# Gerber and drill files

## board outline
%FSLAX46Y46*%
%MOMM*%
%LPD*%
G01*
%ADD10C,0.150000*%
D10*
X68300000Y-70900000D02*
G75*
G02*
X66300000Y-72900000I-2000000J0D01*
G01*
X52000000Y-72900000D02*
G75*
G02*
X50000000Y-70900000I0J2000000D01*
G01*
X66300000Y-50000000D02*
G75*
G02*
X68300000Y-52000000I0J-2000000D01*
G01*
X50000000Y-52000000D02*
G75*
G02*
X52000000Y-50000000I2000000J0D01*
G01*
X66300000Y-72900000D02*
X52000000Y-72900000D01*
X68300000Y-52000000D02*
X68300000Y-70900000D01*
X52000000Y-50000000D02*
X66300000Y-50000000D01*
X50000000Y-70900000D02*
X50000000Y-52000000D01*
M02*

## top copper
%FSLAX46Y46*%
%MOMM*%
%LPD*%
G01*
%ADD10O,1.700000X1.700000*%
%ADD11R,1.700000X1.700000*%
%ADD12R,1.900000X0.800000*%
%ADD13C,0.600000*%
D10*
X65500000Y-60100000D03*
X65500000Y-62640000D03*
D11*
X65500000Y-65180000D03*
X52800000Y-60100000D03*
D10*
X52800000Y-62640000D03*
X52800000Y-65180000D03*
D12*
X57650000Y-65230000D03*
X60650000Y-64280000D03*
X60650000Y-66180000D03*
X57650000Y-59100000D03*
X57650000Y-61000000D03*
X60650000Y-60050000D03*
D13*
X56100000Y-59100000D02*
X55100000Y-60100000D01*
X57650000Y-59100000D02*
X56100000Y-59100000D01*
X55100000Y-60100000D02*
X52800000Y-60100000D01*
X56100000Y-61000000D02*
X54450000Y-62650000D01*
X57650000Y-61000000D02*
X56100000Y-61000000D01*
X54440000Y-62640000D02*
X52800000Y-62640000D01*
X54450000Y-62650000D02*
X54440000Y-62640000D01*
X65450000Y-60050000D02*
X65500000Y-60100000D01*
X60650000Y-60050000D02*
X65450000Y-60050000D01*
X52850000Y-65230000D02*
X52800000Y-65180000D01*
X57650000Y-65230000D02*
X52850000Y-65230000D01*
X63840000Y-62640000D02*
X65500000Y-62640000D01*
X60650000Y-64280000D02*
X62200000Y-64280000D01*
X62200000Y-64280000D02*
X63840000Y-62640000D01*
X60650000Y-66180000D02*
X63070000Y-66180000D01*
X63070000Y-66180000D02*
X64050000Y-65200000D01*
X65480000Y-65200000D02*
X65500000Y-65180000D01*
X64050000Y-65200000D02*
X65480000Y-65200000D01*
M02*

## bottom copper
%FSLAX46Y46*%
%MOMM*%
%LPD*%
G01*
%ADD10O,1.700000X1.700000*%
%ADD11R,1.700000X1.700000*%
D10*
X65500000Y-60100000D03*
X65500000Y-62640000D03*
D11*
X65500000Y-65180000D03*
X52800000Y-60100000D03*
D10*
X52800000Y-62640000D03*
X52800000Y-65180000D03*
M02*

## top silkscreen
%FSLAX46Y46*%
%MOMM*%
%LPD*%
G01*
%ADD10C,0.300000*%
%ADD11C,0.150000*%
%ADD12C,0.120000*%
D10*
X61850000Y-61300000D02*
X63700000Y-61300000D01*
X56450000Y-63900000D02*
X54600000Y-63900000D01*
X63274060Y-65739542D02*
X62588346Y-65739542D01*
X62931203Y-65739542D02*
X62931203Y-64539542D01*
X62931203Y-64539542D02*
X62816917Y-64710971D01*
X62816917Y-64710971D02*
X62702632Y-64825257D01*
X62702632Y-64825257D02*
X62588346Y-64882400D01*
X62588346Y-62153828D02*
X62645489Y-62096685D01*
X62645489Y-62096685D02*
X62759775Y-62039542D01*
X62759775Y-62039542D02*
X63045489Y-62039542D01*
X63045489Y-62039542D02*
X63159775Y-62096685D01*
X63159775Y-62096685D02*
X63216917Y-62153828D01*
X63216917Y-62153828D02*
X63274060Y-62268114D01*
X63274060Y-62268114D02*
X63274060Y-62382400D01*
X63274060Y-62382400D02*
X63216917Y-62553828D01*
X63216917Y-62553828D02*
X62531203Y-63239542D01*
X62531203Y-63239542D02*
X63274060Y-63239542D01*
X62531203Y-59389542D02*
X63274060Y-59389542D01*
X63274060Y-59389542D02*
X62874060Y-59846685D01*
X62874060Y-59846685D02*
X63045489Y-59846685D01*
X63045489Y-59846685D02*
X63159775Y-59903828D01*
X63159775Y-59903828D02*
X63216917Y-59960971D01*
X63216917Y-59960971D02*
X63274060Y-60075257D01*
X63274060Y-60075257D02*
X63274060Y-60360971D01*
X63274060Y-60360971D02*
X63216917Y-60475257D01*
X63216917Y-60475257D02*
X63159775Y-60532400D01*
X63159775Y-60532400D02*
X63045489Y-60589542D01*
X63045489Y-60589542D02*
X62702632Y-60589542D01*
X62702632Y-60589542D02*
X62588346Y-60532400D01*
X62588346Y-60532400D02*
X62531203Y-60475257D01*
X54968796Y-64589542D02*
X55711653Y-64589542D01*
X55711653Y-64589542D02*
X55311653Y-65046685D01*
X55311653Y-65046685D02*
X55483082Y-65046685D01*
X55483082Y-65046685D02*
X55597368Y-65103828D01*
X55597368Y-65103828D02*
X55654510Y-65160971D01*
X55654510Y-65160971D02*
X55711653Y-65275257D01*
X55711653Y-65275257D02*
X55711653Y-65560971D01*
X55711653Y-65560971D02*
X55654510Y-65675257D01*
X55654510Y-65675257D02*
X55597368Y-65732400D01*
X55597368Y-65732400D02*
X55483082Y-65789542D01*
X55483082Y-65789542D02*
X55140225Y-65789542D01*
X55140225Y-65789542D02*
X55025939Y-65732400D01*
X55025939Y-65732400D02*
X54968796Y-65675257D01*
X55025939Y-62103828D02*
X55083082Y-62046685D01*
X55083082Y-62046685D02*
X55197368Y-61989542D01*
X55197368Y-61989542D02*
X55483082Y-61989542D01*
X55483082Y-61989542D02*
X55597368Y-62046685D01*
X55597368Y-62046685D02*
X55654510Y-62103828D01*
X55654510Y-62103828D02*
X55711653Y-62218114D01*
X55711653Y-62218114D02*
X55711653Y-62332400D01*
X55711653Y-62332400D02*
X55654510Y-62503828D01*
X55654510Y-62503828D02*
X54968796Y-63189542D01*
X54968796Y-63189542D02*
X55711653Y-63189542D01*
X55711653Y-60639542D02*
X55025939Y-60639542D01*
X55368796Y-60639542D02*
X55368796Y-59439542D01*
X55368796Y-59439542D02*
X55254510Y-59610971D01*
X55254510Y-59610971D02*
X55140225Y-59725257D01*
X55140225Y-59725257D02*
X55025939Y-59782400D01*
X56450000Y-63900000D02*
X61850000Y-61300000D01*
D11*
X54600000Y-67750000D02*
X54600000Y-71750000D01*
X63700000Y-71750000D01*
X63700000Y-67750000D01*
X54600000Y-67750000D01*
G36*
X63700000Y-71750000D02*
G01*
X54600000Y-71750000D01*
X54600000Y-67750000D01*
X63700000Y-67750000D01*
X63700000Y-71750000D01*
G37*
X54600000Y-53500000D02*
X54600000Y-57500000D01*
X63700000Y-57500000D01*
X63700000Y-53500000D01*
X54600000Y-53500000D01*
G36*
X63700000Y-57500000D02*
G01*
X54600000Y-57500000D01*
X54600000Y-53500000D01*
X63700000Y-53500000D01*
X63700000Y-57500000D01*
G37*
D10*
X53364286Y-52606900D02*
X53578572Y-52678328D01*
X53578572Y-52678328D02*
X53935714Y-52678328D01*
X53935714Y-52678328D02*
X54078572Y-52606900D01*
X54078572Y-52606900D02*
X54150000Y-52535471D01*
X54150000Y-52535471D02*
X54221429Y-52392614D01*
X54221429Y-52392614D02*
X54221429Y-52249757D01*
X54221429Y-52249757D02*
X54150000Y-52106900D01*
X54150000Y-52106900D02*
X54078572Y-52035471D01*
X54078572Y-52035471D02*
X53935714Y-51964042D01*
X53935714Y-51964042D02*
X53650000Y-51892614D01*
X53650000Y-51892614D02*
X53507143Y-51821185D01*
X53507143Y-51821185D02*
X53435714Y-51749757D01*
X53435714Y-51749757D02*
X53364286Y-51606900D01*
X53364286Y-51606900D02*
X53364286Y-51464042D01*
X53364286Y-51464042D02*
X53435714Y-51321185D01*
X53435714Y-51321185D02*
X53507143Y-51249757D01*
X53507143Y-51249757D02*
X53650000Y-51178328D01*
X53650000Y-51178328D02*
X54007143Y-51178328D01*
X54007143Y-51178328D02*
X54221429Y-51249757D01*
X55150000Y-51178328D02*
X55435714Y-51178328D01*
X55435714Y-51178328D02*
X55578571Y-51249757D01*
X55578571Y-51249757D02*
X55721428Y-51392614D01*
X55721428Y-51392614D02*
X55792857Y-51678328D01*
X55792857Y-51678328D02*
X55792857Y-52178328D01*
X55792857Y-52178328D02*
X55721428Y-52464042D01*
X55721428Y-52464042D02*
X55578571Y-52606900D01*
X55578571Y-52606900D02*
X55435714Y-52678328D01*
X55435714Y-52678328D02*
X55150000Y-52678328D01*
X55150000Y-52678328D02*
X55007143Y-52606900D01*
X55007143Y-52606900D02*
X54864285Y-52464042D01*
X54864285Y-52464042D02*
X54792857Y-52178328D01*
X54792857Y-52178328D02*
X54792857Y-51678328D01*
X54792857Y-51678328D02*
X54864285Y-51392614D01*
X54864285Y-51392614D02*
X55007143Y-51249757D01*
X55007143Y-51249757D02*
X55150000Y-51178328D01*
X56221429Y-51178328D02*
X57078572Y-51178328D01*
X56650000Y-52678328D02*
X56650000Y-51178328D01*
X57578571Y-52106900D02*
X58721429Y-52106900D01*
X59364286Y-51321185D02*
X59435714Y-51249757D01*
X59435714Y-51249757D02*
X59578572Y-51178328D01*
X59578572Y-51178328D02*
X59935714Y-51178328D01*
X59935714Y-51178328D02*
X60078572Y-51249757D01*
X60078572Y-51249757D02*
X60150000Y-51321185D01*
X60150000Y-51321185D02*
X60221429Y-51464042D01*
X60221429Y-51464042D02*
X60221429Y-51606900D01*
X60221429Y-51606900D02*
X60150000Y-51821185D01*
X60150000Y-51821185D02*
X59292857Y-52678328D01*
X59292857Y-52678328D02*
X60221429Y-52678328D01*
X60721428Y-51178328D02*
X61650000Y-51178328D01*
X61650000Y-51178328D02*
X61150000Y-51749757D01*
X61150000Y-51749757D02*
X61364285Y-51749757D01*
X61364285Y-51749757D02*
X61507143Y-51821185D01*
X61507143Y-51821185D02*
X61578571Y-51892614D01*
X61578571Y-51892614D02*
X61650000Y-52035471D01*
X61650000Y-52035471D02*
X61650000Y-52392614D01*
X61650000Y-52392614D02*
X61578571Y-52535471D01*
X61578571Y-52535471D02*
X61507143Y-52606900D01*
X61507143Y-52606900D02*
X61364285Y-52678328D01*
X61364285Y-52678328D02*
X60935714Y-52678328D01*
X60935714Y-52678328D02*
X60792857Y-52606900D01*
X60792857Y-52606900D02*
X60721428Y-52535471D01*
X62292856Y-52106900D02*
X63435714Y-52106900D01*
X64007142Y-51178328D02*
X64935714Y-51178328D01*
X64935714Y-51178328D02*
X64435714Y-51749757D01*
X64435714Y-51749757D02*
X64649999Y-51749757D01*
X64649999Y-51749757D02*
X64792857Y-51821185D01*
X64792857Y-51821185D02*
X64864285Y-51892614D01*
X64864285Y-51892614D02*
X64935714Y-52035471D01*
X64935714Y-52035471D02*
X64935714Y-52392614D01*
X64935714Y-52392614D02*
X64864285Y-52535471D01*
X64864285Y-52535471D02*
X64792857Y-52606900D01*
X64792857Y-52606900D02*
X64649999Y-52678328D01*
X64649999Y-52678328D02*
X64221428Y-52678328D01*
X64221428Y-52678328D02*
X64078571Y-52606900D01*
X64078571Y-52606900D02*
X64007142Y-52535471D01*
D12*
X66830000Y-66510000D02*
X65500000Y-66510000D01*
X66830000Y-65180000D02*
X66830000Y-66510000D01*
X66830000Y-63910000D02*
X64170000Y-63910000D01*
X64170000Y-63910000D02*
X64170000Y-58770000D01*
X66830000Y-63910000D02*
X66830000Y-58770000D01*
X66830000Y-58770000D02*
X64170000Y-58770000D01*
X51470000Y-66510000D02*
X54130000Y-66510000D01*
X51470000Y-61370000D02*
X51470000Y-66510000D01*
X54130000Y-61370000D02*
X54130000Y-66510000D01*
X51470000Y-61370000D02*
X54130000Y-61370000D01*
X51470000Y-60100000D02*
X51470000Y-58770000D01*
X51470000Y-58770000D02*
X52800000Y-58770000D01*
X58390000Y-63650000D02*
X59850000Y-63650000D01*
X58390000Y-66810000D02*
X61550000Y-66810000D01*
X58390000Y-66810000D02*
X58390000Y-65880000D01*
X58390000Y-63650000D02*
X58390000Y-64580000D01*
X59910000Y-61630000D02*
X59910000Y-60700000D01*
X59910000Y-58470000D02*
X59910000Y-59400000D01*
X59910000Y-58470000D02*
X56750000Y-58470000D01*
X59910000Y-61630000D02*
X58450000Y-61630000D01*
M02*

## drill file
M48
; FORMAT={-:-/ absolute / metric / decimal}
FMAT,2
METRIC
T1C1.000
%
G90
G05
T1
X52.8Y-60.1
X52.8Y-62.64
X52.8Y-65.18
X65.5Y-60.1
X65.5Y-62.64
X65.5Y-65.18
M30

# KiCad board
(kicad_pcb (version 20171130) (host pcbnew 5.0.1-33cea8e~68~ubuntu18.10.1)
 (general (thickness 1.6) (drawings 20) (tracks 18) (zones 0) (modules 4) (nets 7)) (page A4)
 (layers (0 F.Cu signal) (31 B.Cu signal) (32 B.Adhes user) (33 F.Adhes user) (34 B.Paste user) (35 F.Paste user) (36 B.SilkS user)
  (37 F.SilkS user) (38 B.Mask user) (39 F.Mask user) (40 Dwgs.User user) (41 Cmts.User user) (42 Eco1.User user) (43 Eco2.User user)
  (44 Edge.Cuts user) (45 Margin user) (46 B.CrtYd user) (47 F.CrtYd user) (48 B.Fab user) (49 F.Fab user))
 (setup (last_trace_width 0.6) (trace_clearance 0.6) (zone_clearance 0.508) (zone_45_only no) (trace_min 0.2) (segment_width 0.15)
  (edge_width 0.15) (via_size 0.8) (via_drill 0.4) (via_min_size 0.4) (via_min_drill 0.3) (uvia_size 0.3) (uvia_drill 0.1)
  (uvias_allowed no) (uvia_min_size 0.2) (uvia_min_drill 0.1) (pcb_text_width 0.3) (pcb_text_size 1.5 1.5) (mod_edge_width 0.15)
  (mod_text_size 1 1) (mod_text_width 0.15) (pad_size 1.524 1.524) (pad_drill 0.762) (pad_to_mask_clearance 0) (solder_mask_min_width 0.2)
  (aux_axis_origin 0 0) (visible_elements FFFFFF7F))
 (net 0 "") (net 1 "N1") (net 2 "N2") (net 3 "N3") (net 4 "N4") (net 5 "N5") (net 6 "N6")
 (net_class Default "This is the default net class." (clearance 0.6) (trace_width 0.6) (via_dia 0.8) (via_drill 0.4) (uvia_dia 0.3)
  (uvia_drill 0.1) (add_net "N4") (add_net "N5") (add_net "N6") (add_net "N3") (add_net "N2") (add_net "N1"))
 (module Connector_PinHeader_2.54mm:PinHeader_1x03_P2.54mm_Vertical (layer F.Cu) (at 65.5 65.18 180)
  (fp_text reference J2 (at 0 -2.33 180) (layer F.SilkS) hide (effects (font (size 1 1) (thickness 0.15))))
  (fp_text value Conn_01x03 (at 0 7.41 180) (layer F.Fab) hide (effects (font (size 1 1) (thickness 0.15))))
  (fp_line (start -1.33 -1.33) (end 0 -1.33) (layer F.SilkS) (width 0.12))
  (fp_line (start -1.33 0) (end -1.33 -1.33) (layer F.SilkS) (width 0.12))
  (fp_line (start -1.33 1.27) (end 1.33 1.27) (layer F.SilkS) (width 0.12))
  (fp_line (start 1.33 1.27) (end 1.33 6.41) (layer F.SilkS) (width 0.12))
  (fp_line (start -1.33 1.27) (end -1.33 6.41) (layer F.SilkS) (width 0.12))
  (fp_line (start -1.33 6.41) (end 1.33 6.41) (layer F.SilkS) (width 0.12))
  (pad 3 thru_hole oval (at 0 5.08 180) (size 1.7 1.7) (drill 1) (layers *.Cu *.Mask) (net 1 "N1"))
  (pad 2 thru_hole oval (at 0 2.54 180) (size 1.7 1.7) (drill 1) (layers *.Cu *.Mask) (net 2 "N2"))
  (pad 1 thru_hole rect (at 0 0 180) (size 1.7 1.7) (drill 1) (layers *.Cu *.Mask) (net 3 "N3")))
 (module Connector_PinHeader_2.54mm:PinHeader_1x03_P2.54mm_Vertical (layer F.Cu) (at 52.8 60.1)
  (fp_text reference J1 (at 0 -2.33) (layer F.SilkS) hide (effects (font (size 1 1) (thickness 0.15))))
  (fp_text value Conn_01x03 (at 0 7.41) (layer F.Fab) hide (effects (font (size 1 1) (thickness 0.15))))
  (fp_line (start -1.33 6.41) (end 1.33 6.41) (layer F.SilkS) (width 0.12))
  (fp_line (start -1.33 1.27) (end -1.33 6.41) (layer F.SilkS) (width 0.12))
  (fp_line (start 1.33 1.27) (end 1.33 6.41) (layer F.SilkS) (width 0.12))
  (fp_line (start -1.33 1.27) (end 1.33 1.27) (layer F.SilkS) (width 0.12))
  (fp_line (start -1.33 0) (end -1.33 -1.33) (layer F.SilkS) (width 0.12))
  (fp_line (start -1.33 -1.33) (end 0 -1.33) (layer F.SilkS) (width 0.12))
  (pad 1 thru_hole rect (at 0 0) (size 1.7 1.7) (drill 1) (layers *.Cu *.Mask) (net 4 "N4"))
  (pad 2 thru_hole oval (at 0 2.54) (size 1.7 1.7) (drill 1) (layers *.Cu *.Mask) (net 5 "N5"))
  (pad 3 thru_hole oval (at 0 5.08) (size 1.7 1.7) (drill 1) (layers *.Cu *.Mask) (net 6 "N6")))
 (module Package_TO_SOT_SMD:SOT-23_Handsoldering (layer F.Cu) (at 59.15 65.23 180)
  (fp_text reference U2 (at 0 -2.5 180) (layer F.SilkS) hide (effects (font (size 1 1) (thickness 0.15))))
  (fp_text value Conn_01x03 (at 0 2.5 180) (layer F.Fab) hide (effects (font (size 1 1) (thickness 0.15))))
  (fp_line (start 0.76 1.58) (end -0.7 1.58) (layer F.SilkS) (width 0.12))
  (fp_line (start 0.76 -1.58) (end -2.4 -1.58) (layer F.SilkS) (width 0.12))
  (fp_line (start 0.76 -1.58) (end 0.76 -0.65) (layer F.SilkS) (width 0.12))
  (fp_line (start 0.76 1.58) (end 0.76 0.65) (layer F.SilkS) (width 0.12))
  (pad 3 smd rect (at 1.5 0 180) (size 1.9 0.8) (layers F.Cu F.Paste F.Mask) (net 6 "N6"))
  (pad 2 smd rect (at -1.5 0.95 180) (size 1.9 0.8) (layers F.Cu F.Paste F.Mask) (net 2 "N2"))
  (pad 1 smd rect (at -1.5 -0.95 180) (size 1.9 0.8) (layers F.Cu F.Paste F.Mask) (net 3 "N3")))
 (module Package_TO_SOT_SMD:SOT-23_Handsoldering (layer F.Cu) (at 59.15 60.05)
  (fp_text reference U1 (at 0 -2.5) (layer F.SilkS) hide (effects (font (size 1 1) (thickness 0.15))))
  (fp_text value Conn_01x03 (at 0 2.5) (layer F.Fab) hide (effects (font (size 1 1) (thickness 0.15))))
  (fp_line (start 0.76 1.58) (end 0.76 0.65) (layer F.SilkS) (width 0.12))
  (fp_line (start 0.76 -1.58) (end 0.76 -0.65) (layer F.SilkS) (width 0.12))
  (fp_line (start 0.76 -1.58) (end -2.4 -1.58) (layer F.SilkS) (width 0.12))
  (fp_line (start 0.76 1.58) (end -0.7 1.58) (layer F.SilkS) (width 0.12))
  (pad 1 smd rect (at -1.5 -0.95) (size 1.9 0.8) (layers F.Cu F.Paste F.Mask) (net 4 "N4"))
  (pad 2 smd rect (at -1.5 0.95) (size 1.9 0.8) (layers F.Cu F.Paste F.Mask) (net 5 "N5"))
  (pad 3 smd rect (at 1.5 0) (size 1.9 0.8) (layers F.Cu F.Paste F.Mask) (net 1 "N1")))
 (gr_arc (start 66.3 70.9) (end 66.3 72.9) (angle -90) (layer Edge.Cuts) (width 0.15))
 (gr_arc (start 52 70.9) (end 50 70.9) (angle -90) (layer Edge.Cuts) (width 0.15))
 (gr_arc (start 66.3 52) (end 68.3 52) (angle -90) (layer Edge.Cuts) (width 0.15))
 (gr_arc (start 52 52) (end 52 50) (angle -90) (layer Edge.Cuts) (width 0.15))
 (gr_line (start 61.85 61.3) (end 63.7 61.3) (layer F.SilkS) (width 0.3))
 (gr_line (start 56.45 63.9) (end 54.6 63.9) (layer F.SilkS) (width 0.3))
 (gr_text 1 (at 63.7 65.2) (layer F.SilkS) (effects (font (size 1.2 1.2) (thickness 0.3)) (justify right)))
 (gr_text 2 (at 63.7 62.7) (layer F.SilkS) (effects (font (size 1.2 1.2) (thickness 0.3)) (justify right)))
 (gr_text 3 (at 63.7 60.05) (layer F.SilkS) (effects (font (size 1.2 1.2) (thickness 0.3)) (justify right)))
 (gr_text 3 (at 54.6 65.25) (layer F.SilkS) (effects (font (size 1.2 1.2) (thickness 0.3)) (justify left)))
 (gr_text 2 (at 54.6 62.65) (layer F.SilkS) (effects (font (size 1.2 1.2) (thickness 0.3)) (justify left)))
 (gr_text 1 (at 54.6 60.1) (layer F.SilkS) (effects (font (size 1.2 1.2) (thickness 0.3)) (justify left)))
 (gr_line (start 56.45 63.9) (end 61.85 61.3) (layer F.SilkS) (width 0.3))
 (gr_line (start 66.3 72.9) (end 52 72.9) (layer Edge.Cuts) (width 0.15))
 (gr_poly (pts (xy 54.6 67.75) (xy 54.6 71.75) (xy 63.7 71.75) (xy 63.7 67.75)) (layer F.SilkS) (width 0.15))
 (gr_poly (pts (xy 54.6 53.5) (xy 54.6 57.5) (xy 63.7 57.5) (xy 63.7 53.5)) (layer F.SilkS) (width 0.15))
 (gr_line (start 68.3 52) (end 68.3 70.9) (layer Edge.Cuts) (width 0.15))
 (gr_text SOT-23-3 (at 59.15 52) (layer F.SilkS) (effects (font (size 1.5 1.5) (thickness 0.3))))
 (gr_line (start 52 50) (end 66.3 50) (layer Edge.Cuts) (width 0.15))
 (gr_line (start 50 70.9) (end 50 52) (layer Edge.Cuts) (width 0.15))
 (segment (start 56.1 59.1) (end 55.1 60.1) (width 0.6) (layer F.Cu) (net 4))
 (segment (start 57.65 59.1) (end 56.1 59.1) (width 0.6) (layer F.Cu) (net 4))
 (segment (start 55.1 60.1) (end 52.8 60.1) (width 0.6) (layer F.Cu) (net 4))
 (segment (start 56.1 61) (end 54.45 62.65) (width 0.6) (layer F.Cu) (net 5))
 (segment (start 57.65 61) (end 56.1 61) (width 0.6) (layer F.Cu) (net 5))
 (segment (start 54.44 62.64) (end 52.8 62.64) (width 0.6) (layer F.Cu) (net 5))
 (segment (start 54.45 62.65) (end 54.44 62.64) (width 0.6) (layer F.Cu) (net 5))
 (segment (start 65.45 60.05) (end 65.5 60.1) (width 0.6) (layer F.Cu) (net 1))
 (segment (start 60.65 60.05) (end 65.45 60.05) (width 0.6) (layer F.Cu) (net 1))
 (segment (start 52.85 65.23) (end 52.8 65.18) (width 0.6) (layer F.Cu) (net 6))
 (segment (start 57.65 65.23) (end 52.85 65.23) (width 0.6) (layer F.Cu) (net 6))
 (segment (start 63.84 62.64) (end 65.5 62.64) (width 0.6) (layer F.Cu) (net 2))
 (segment (start 60.65 64.28) (end 62.2 64.28) (width 0.6) (layer F.Cu) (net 2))
 (segment (start 62.2 64.28) (end 63.84 62.64) (width 0.6) (layer F.Cu) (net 2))
 (segment (start 60.65 66.18) (end 63.07 66.18) (width 0.6) (layer F.Cu) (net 3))
 (segment (start 63.07 66.18) (end 64.05 65.2) (width 0.6) (layer F.Cu) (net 3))
 (segment (start 65.48 65.2) (end 65.5 65.18) (width 0.6) (layer F.Cu) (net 3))
 (segment (start 64.05 65.2) (end 65.48 65.2) (width 0.6) (layer F.Cu) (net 3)))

